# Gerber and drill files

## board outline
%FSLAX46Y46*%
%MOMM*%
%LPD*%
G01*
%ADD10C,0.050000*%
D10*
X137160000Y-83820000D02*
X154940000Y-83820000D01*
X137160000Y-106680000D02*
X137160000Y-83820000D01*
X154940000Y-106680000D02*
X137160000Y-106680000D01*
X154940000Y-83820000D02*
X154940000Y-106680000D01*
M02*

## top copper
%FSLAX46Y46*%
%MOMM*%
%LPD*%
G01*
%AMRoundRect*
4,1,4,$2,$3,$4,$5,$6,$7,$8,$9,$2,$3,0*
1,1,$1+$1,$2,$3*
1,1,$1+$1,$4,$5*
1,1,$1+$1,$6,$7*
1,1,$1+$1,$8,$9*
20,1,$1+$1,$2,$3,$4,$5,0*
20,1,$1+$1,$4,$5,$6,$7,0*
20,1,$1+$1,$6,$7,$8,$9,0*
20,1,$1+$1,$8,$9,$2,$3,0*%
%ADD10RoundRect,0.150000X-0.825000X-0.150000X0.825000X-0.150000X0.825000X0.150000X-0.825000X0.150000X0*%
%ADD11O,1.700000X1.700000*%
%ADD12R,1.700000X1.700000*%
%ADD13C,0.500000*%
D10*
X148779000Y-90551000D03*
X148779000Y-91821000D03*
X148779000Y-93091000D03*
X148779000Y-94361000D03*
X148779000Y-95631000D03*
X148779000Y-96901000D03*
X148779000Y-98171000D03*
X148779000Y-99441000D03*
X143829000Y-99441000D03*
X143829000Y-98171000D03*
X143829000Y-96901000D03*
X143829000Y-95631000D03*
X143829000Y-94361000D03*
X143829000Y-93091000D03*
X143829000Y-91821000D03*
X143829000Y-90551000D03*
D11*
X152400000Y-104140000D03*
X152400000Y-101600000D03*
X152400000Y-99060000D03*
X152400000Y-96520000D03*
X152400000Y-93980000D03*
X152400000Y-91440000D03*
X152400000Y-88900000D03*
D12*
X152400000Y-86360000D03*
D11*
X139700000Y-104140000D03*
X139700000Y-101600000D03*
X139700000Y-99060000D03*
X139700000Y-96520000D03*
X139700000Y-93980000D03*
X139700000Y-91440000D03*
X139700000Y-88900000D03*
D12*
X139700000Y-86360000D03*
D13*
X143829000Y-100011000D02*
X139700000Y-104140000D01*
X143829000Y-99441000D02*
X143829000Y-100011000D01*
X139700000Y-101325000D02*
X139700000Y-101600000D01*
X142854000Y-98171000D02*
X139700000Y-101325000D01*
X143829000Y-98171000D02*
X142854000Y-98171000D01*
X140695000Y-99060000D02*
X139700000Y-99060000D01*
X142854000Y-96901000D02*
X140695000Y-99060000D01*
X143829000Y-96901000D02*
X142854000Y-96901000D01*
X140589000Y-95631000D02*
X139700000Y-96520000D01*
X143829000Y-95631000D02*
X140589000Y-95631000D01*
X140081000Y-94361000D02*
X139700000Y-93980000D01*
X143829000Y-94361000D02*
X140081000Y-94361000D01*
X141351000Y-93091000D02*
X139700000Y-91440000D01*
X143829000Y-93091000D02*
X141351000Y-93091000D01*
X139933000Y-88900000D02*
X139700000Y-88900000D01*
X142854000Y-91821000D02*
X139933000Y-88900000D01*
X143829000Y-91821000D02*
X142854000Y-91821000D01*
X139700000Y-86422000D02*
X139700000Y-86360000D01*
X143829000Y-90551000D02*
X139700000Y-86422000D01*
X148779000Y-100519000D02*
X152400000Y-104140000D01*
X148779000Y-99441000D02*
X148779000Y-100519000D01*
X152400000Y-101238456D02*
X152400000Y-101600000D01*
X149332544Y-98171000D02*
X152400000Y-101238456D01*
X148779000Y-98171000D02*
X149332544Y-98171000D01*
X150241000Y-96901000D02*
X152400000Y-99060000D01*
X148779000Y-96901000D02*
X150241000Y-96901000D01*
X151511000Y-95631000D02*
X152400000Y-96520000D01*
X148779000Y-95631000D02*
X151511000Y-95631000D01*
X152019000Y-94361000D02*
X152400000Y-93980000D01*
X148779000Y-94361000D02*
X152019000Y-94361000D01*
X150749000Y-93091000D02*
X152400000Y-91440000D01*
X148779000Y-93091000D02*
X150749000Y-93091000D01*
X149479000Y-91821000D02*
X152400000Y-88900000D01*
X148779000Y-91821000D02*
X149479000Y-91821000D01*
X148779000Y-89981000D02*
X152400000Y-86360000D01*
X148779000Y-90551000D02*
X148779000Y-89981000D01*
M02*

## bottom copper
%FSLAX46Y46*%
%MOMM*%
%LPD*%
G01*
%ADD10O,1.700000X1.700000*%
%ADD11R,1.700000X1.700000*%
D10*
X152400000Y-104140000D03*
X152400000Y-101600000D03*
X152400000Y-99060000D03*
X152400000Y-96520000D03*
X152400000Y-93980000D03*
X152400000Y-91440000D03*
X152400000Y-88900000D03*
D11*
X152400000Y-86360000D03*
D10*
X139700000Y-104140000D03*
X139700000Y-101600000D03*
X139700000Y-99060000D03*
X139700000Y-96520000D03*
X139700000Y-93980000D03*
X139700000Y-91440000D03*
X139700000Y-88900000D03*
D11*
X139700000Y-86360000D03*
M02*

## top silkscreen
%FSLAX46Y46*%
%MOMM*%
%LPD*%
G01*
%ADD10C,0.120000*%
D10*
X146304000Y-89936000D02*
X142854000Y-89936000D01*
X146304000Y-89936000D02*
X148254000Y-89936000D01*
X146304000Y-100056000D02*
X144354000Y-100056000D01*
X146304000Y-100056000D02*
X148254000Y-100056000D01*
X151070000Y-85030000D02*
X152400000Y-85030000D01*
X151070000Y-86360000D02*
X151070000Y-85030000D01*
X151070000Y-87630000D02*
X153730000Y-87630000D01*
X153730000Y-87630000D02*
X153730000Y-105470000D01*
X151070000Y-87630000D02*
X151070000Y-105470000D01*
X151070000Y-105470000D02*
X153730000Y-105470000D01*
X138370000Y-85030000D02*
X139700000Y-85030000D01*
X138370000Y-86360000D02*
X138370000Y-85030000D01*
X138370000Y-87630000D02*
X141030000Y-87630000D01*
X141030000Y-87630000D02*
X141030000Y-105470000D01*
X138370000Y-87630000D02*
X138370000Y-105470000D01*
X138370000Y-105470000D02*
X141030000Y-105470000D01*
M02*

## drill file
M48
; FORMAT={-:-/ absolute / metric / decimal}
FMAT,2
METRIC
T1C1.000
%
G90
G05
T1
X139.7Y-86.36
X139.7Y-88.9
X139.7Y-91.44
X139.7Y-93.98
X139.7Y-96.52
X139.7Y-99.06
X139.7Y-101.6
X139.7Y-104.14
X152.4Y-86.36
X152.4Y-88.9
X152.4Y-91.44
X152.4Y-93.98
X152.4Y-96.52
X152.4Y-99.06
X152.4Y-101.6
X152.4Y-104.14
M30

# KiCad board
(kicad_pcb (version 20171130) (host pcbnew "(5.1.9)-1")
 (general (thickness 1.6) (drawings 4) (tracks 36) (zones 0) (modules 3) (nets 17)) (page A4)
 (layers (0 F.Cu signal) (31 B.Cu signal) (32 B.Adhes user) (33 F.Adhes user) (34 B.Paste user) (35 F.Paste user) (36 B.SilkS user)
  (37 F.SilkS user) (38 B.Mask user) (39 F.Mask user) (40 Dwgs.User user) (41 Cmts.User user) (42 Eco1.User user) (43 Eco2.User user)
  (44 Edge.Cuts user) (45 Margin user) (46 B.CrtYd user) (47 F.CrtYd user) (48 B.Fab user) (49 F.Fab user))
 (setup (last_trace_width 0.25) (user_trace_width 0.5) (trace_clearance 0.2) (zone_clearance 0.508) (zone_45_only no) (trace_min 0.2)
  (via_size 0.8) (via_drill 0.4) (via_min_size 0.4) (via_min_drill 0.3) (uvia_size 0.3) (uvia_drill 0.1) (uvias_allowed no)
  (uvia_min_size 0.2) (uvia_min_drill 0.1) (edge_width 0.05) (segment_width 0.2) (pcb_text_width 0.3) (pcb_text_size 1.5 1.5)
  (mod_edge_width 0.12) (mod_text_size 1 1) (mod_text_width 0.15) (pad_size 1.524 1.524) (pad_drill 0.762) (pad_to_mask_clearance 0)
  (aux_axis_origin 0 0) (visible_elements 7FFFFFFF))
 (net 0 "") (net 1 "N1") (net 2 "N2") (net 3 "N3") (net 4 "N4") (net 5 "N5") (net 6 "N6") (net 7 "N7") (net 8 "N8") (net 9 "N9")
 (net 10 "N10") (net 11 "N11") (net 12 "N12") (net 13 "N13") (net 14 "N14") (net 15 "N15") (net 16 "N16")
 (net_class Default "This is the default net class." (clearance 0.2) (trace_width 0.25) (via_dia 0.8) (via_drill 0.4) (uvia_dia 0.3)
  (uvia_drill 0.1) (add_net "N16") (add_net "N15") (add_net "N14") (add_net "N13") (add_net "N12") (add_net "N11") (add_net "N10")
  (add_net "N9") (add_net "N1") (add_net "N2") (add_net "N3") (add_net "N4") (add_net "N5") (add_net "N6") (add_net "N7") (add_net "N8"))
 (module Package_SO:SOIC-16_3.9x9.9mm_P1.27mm (layer F.Cu) (at 146.304 94.996)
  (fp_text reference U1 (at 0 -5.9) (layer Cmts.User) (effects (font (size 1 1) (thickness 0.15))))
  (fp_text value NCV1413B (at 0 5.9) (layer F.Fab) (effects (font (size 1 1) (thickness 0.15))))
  (fp_line (start 0 -5.06) (end -3.45 -5.06) (layer F.SilkS) (width 0.12))
  (fp_line (start 0 -5.06) (end 1.95 -5.06) (layer F.SilkS) (width 0.12))
  (fp_line (start 0 5.06) (end -1.95 5.06) (layer F.SilkS) (width 0.12))
  (fp_line (start 0 5.06) (end 1.95 5.06) (layer F.SilkS) (width 0.12))
  (pad 16 smd roundrect (at 2.475 -4.445) (size 1.95 0.6) (layers F.Cu F.Paste F.Mask) (roundrect_rratio 0.25) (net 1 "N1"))
  (pad 15 smd roundrect (at 2.475 -3.175) (size 1.95 0.6) (layers F.Cu F.Paste F.Mask) (roundrect_rratio 0.25) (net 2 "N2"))
  (pad 14 smd roundrect (at 2.475 -1.905) (size 1.95 0.6) (layers F.Cu F.Paste F.Mask) (roundrect_rratio 0.25) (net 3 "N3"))
  (pad 13 smd roundrect (at 2.475 -0.635) (size 1.95 0.6) (layers F.Cu F.Paste F.Mask) (roundrect_rratio 0.25) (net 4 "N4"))
  (pad 12 smd roundrect (at 2.475 0.635) (size 1.95 0.6) (layers F.Cu F.Paste F.Mask) (roundrect_rratio 0.25) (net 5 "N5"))
  (pad 11 smd roundrect (at 2.475 1.905) (size 1.95 0.6) (layers F.Cu F.Paste F.Mask) (roundrect_rratio 0.25) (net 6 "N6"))
  (pad 10 smd roundrect (at 2.475 3.175) (size 1.95 0.6) (layers F.Cu F.Paste F.Mask) (roundrect_rratio 0.25) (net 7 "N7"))
  (pad 9 smd roundrect (at 2.475 4.445) (size 1.95 0.6) (layers F.Cu F.Paste F.Mask) (roundrect_rratio 0.25) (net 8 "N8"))
  (pad 8 smd roundrect (at -2.475 4.445) (size 1.95 0.6) (layers F.Cu F.Paste F.Mask) (roundrect_rratio 0.25) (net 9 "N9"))
  (pad 7 smd roundrect (at -2.475 3.175) (size 1.95 0.6) (layers F.Cu F.Paste F.Mask) (roundrect_rratio 0.25) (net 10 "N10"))
  (pad 6 smd roundrect (at -2.475 1.905) (size 1.95 0.6) (layers F.Cu F.Paste F.Mask) (roundrect_rratio 0.25) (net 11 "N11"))
  (pad 5 smd roundrect (at -2.475 0.635) (size 1.95 0.6) (layers F.Cu F.Paste F.Mask) (roundrect_rratio 0.25) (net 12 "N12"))
  (pad 4 smd roundrect (at -2.475 -0.635) (size 1.95 0.6) (layers F.Cu F.Paste F.Mask) (roundrect_rratio 0.25) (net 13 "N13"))
  (pad 3 smd roundrect (at -2.475 -1.905) (size 1.95 0.6) (layers F.Cu F.Paste F.Mask) (roundrect_rratio 0.25) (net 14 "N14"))
  (pad 2 smd roundrect (at -2.475 -3.175) (size 1.95 0.6) (layers F.Cu F.Paste F.Mask) (roundrect_rratio 0.25) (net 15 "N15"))
  (pad 1 smd roundrect (at -2.475 -4.445) (size 1.95 0.6) (layers F.Cu F.Paste F.Mask) (roundrect_rratio 0.25) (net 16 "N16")))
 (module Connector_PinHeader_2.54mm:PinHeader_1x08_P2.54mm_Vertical (layer F.Cu) (at 152.4 86.36)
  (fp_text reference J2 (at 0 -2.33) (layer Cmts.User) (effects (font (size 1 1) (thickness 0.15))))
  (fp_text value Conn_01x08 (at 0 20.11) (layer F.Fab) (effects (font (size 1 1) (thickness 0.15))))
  (fp_line (start -1.33 -1.33) (end 0 -1.33) (layer F.SilkS) (width 0.12))
  (fp_line (start -1.33 0) (end -1.33 -1.33) (layer F.SilkS) (width 0.12))
  (fp_line (start -1.33 1.27) (end 1.33 1.27) (layer F.SilkS) (width 0.12))
  (fp_line (start 1.33 1.27) (end 1.33 19.11) (layer F.SilkS) (width 0.12))
  (fp_line (start -1.33 1.27) (end -1.33 19.11) (layer F.SilkS) (width 0.12))
  (fp_line (start -1.33 19.11) (end 1.33 19.11) (layer F.SilkS) (width 0.12))
  (pad 8 thru_hole oval (at 0 17.78) (size 1.7 1.7) (drill 1) (layers *.Cu *.Mask) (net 8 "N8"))
  (pad 7 thru_hole oval (at 0 15.24) (size 1.7 1.7) (drill 1) (layers *.Cu *.Mask) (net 7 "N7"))
  (pad 6 thru_hole oval (at 0 12.7) (size 1.7 1.7) (drill 1) (layers *.Cu *.Mask) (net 6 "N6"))
  (pad 5 thru_hole oval (at 0 10.16) (size 1.7 1.7) (drill 1) (layers *.Cu *.Mask) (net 5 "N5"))
  (pad 4 thru_hole oval (at 0 7.62) (size 1.7 1.7) (drill 1) (layers *.Cu *.Mask) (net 4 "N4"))
  (pad 3 thru_hole oval (at 0 5.08) (size 1.7 1.7) (drill 1) (layers *.Cu *.Mask) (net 3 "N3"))
  (pad 2 thru_hole oval (at 0 2.54) (size 1.7 1.7) (drill 1) (layers *.Cu *.Mask) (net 2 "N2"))
  (pad 1 thru_hole rect (at 0 0) (size 1.7 1.7) (drill 1) (layers *.Cu *.Mask) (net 1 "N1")))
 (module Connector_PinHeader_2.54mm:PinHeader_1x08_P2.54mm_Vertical (layer F.Cu) (at 139.7 86.36)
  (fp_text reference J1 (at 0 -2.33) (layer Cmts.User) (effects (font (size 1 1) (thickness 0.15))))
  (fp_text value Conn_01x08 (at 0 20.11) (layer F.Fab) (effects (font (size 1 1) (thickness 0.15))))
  (fp_line (start -1.33 -1.33) (end 0 -1.33) (layer F.SilkS) (width 0.12))
  (fp_line (start -1.33 0) (end -1.33 -1.33) (layer F.SilkS) (width 0.12))
  (fp_line (start -1.33 1.27) (end 1.33 1.27) (layer F.SilkS) (width 0.12))
  (fp_line (start 1.33 1.27) (end 1.33 19.11) (layer F.SilkS) (width 0.12))
  (fp_line (start -1.33 1.27) (end -1.33 19.11) (layer F.SilkS) (width 0.12))
  (fp_line (start -1.33 19.11) (end 1.33 19.11) (layer F.SilkS) (width 0.12))
  (pad 8 thru_hole oval (at 0 17.78) (size 1.7 1.7) (drill 1) (layers *.Cu *.Mask) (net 9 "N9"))
  (pad 7 thru_hole oval (at 0 15.24) (size 1.7 1.7) (drill 1) (layers *.Cu *.Mask) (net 10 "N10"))
  (pad 6 thru_hole oval (at 0 12.7) (size 1.7 1.7) (drill 1) (layers *.Cu *.Mask) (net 11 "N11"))
  (pad 5 thru_hole oval (at 0 10.16) (size 1.7 1.7) (drill 1) (layers *.Cu *.Mask) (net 12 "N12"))
  (pad 4 thru_hole oval (at 0 7.62) (size 1.7 1.7) (drill 1) (layers *.Cu *.Mask) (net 13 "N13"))
  (pad 3 thru_hole oval (at 0 5.08) (size 1.7 1.7) (drill 1) (layers *.Cu *.Mask) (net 14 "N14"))
  (pad 2 thru_hole oval (at 0 2.54) (size 1.7 1.7) (drill 1) (layers *.Cu *.Mask) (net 15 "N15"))
  (pad 1 thru_hole rect (at 0 0) (size 1.7 1.7) (drill 1) (layers *.Cu *.Mask) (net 16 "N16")))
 (gr_line (start 137.16 83.82) (end 154.94 83.82) (layer Edge.Cuts) (width 0.05))
 (gr_line (start 137.16 106.68) (end 137.16 83.82) (layer Edge.Cuts) (width 0.05))
 (gr_line (start 154.94 106.68) (end 137.16 106.68) (layer Edge.Cuts) (width 0.05))
 (gr_line (start 154.94 83.82) (end 154.94 106.68) (layer Edge.Cuts) (width 0.05))
 (segment (start 143.829 100.011) (end 139.7 104.14) (width 0.5) (layer F.Cu) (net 9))
 (segment (start 143.829 99.441) (end 143.829 100.011) (width 0.5) (layer F.Cu) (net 9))
 (segment (start 139.7 101.325) (end 139.7 101.6) (width 0.5) (layer F.Cu) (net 10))
 (segment (start 142.854 98.171) (end 139.7 101.325) (width 0.5) (layer F.Cu) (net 10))
 (segment (start 143.829 98.171) (end 142.854 98.171) (width 0.5) (layer F.Cu) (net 10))
 (segment (start 140.695 99.06) (end 139.7 99.06) (width 0.5) (layer F.Cu) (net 11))
 (segment (start 142.854 96.901) (end 140.695 99.06) (width 0.5) (layer F.Cu) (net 11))
 (segment (start 143.829 96.901) (end 142.854 96.901) (width 0.5) (layer F.Cu) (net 11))
 (segment (start 140.589 95.631) (end 139.7 96.52) (width 0.5) (layer F.Cu) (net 12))
 (segment (start 143.829 95.631) (end 140.589 95.631) (width 0.5) (layer F.Cu) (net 12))
 (segment (start 140.081 94.361) (end 139.7 93.98) (width 0.5) (layer F.Cu) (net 13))
 (segment (start 143.829 94.361) (end 140.081 94.361) (width 0.5) (layer F.Cu) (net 13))
 (segment (start 141.351 93.091) (end 139.7 91.44) (width 0.5) (layer F.Cu) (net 14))
 (segment (start 143.829 93.091) (end 141.351 93.091) (width 0.5) (layer F.Cu) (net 14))
 (segment (start 139.933 88.9) (end 139.7 88.9) (width 0.5) (layer F.Cu) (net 15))
 (segment (start 142.854 91.821) (end 139.933 88.9) (width 0.5) (layer F.Cu) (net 15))
 (segment (start 143.829 91.821) (end 142.854 91.821) (width 0.5) (layer F.Cu) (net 15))
 (segment (start 139.7 86.422) (end 139.7 86.36) (width 0.5) (layer F.Cu) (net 16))
 (segment (start 143.829 90.551) (end 139.7 86.422) (width 0.5) (layer F.Cu) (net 16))
 (segment (start 148.779 100.519) (end 152.4 104.14) (width 0.5) (layer F.Cu) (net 8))
 (segment (start 148.779 99.441) (end 148.779 100.519) (width 0.5) (layer F.Cu) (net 8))
 (segment (start 152.4 101.238456) (end 152.4 101.6) (width 0.5) (layer F.Cu) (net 7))
 (segment (start 149.332544 98.171) (end 152.4 101.238456) (width 0.5) (layer F.Cu) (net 7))
 (segment (start 148.779 98.171) (end 149.332544 98.171) (width 0.5) (layer F.Cu) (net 7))
 (segment (start 150.241 96.901) (end 152.4 99.06) (width 0.5) (layer F.Cu) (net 6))
 (segment (start 148.779 96.901) (end 150.241 96.901) (width 0.5) (layer F.Cu) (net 6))
 (segment (start 151.511 95.631) (end 152.4 96.52) (width 0.5) (layer F.Cu) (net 5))
 (segment (start 148.779 95.631) (end 151.511 95.631) (width 0.5) (layer F.Cu) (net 5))
 (segment (start 152.019 94.361) (end 152.4 93.98) (width 0.5) (layer F.Cu) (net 4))
 (segment (start 148.779 94.361) (end 152.019 94.361) (width 0.5) (layer F.Cu) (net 4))
 (segment (start 150.749 93.091) (end 152.4 91.44) (width 0.5) (layer F.Cu) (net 3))
 (segment (start 148.779 93.091) (end 150.749 93.091) (width 0.5) (layer F.Cu) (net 3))
 (segment (start 149.479 91.821) (end 152.4 88.9) (width 0.5) (layer F.Cu) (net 2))
 (segment (start 148.779 91.821) (end 149.479 91.821) (width 0.5) (layer F.Cu) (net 2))
 (segment (start 148.779 89.981) (end 152.4 86.36) (width 0.5) (layer F.Cu) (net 1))
 (segment (start 148.779 90.551) (end 148.779 89.981) (width 0.5) (layer F.Cu) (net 1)))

